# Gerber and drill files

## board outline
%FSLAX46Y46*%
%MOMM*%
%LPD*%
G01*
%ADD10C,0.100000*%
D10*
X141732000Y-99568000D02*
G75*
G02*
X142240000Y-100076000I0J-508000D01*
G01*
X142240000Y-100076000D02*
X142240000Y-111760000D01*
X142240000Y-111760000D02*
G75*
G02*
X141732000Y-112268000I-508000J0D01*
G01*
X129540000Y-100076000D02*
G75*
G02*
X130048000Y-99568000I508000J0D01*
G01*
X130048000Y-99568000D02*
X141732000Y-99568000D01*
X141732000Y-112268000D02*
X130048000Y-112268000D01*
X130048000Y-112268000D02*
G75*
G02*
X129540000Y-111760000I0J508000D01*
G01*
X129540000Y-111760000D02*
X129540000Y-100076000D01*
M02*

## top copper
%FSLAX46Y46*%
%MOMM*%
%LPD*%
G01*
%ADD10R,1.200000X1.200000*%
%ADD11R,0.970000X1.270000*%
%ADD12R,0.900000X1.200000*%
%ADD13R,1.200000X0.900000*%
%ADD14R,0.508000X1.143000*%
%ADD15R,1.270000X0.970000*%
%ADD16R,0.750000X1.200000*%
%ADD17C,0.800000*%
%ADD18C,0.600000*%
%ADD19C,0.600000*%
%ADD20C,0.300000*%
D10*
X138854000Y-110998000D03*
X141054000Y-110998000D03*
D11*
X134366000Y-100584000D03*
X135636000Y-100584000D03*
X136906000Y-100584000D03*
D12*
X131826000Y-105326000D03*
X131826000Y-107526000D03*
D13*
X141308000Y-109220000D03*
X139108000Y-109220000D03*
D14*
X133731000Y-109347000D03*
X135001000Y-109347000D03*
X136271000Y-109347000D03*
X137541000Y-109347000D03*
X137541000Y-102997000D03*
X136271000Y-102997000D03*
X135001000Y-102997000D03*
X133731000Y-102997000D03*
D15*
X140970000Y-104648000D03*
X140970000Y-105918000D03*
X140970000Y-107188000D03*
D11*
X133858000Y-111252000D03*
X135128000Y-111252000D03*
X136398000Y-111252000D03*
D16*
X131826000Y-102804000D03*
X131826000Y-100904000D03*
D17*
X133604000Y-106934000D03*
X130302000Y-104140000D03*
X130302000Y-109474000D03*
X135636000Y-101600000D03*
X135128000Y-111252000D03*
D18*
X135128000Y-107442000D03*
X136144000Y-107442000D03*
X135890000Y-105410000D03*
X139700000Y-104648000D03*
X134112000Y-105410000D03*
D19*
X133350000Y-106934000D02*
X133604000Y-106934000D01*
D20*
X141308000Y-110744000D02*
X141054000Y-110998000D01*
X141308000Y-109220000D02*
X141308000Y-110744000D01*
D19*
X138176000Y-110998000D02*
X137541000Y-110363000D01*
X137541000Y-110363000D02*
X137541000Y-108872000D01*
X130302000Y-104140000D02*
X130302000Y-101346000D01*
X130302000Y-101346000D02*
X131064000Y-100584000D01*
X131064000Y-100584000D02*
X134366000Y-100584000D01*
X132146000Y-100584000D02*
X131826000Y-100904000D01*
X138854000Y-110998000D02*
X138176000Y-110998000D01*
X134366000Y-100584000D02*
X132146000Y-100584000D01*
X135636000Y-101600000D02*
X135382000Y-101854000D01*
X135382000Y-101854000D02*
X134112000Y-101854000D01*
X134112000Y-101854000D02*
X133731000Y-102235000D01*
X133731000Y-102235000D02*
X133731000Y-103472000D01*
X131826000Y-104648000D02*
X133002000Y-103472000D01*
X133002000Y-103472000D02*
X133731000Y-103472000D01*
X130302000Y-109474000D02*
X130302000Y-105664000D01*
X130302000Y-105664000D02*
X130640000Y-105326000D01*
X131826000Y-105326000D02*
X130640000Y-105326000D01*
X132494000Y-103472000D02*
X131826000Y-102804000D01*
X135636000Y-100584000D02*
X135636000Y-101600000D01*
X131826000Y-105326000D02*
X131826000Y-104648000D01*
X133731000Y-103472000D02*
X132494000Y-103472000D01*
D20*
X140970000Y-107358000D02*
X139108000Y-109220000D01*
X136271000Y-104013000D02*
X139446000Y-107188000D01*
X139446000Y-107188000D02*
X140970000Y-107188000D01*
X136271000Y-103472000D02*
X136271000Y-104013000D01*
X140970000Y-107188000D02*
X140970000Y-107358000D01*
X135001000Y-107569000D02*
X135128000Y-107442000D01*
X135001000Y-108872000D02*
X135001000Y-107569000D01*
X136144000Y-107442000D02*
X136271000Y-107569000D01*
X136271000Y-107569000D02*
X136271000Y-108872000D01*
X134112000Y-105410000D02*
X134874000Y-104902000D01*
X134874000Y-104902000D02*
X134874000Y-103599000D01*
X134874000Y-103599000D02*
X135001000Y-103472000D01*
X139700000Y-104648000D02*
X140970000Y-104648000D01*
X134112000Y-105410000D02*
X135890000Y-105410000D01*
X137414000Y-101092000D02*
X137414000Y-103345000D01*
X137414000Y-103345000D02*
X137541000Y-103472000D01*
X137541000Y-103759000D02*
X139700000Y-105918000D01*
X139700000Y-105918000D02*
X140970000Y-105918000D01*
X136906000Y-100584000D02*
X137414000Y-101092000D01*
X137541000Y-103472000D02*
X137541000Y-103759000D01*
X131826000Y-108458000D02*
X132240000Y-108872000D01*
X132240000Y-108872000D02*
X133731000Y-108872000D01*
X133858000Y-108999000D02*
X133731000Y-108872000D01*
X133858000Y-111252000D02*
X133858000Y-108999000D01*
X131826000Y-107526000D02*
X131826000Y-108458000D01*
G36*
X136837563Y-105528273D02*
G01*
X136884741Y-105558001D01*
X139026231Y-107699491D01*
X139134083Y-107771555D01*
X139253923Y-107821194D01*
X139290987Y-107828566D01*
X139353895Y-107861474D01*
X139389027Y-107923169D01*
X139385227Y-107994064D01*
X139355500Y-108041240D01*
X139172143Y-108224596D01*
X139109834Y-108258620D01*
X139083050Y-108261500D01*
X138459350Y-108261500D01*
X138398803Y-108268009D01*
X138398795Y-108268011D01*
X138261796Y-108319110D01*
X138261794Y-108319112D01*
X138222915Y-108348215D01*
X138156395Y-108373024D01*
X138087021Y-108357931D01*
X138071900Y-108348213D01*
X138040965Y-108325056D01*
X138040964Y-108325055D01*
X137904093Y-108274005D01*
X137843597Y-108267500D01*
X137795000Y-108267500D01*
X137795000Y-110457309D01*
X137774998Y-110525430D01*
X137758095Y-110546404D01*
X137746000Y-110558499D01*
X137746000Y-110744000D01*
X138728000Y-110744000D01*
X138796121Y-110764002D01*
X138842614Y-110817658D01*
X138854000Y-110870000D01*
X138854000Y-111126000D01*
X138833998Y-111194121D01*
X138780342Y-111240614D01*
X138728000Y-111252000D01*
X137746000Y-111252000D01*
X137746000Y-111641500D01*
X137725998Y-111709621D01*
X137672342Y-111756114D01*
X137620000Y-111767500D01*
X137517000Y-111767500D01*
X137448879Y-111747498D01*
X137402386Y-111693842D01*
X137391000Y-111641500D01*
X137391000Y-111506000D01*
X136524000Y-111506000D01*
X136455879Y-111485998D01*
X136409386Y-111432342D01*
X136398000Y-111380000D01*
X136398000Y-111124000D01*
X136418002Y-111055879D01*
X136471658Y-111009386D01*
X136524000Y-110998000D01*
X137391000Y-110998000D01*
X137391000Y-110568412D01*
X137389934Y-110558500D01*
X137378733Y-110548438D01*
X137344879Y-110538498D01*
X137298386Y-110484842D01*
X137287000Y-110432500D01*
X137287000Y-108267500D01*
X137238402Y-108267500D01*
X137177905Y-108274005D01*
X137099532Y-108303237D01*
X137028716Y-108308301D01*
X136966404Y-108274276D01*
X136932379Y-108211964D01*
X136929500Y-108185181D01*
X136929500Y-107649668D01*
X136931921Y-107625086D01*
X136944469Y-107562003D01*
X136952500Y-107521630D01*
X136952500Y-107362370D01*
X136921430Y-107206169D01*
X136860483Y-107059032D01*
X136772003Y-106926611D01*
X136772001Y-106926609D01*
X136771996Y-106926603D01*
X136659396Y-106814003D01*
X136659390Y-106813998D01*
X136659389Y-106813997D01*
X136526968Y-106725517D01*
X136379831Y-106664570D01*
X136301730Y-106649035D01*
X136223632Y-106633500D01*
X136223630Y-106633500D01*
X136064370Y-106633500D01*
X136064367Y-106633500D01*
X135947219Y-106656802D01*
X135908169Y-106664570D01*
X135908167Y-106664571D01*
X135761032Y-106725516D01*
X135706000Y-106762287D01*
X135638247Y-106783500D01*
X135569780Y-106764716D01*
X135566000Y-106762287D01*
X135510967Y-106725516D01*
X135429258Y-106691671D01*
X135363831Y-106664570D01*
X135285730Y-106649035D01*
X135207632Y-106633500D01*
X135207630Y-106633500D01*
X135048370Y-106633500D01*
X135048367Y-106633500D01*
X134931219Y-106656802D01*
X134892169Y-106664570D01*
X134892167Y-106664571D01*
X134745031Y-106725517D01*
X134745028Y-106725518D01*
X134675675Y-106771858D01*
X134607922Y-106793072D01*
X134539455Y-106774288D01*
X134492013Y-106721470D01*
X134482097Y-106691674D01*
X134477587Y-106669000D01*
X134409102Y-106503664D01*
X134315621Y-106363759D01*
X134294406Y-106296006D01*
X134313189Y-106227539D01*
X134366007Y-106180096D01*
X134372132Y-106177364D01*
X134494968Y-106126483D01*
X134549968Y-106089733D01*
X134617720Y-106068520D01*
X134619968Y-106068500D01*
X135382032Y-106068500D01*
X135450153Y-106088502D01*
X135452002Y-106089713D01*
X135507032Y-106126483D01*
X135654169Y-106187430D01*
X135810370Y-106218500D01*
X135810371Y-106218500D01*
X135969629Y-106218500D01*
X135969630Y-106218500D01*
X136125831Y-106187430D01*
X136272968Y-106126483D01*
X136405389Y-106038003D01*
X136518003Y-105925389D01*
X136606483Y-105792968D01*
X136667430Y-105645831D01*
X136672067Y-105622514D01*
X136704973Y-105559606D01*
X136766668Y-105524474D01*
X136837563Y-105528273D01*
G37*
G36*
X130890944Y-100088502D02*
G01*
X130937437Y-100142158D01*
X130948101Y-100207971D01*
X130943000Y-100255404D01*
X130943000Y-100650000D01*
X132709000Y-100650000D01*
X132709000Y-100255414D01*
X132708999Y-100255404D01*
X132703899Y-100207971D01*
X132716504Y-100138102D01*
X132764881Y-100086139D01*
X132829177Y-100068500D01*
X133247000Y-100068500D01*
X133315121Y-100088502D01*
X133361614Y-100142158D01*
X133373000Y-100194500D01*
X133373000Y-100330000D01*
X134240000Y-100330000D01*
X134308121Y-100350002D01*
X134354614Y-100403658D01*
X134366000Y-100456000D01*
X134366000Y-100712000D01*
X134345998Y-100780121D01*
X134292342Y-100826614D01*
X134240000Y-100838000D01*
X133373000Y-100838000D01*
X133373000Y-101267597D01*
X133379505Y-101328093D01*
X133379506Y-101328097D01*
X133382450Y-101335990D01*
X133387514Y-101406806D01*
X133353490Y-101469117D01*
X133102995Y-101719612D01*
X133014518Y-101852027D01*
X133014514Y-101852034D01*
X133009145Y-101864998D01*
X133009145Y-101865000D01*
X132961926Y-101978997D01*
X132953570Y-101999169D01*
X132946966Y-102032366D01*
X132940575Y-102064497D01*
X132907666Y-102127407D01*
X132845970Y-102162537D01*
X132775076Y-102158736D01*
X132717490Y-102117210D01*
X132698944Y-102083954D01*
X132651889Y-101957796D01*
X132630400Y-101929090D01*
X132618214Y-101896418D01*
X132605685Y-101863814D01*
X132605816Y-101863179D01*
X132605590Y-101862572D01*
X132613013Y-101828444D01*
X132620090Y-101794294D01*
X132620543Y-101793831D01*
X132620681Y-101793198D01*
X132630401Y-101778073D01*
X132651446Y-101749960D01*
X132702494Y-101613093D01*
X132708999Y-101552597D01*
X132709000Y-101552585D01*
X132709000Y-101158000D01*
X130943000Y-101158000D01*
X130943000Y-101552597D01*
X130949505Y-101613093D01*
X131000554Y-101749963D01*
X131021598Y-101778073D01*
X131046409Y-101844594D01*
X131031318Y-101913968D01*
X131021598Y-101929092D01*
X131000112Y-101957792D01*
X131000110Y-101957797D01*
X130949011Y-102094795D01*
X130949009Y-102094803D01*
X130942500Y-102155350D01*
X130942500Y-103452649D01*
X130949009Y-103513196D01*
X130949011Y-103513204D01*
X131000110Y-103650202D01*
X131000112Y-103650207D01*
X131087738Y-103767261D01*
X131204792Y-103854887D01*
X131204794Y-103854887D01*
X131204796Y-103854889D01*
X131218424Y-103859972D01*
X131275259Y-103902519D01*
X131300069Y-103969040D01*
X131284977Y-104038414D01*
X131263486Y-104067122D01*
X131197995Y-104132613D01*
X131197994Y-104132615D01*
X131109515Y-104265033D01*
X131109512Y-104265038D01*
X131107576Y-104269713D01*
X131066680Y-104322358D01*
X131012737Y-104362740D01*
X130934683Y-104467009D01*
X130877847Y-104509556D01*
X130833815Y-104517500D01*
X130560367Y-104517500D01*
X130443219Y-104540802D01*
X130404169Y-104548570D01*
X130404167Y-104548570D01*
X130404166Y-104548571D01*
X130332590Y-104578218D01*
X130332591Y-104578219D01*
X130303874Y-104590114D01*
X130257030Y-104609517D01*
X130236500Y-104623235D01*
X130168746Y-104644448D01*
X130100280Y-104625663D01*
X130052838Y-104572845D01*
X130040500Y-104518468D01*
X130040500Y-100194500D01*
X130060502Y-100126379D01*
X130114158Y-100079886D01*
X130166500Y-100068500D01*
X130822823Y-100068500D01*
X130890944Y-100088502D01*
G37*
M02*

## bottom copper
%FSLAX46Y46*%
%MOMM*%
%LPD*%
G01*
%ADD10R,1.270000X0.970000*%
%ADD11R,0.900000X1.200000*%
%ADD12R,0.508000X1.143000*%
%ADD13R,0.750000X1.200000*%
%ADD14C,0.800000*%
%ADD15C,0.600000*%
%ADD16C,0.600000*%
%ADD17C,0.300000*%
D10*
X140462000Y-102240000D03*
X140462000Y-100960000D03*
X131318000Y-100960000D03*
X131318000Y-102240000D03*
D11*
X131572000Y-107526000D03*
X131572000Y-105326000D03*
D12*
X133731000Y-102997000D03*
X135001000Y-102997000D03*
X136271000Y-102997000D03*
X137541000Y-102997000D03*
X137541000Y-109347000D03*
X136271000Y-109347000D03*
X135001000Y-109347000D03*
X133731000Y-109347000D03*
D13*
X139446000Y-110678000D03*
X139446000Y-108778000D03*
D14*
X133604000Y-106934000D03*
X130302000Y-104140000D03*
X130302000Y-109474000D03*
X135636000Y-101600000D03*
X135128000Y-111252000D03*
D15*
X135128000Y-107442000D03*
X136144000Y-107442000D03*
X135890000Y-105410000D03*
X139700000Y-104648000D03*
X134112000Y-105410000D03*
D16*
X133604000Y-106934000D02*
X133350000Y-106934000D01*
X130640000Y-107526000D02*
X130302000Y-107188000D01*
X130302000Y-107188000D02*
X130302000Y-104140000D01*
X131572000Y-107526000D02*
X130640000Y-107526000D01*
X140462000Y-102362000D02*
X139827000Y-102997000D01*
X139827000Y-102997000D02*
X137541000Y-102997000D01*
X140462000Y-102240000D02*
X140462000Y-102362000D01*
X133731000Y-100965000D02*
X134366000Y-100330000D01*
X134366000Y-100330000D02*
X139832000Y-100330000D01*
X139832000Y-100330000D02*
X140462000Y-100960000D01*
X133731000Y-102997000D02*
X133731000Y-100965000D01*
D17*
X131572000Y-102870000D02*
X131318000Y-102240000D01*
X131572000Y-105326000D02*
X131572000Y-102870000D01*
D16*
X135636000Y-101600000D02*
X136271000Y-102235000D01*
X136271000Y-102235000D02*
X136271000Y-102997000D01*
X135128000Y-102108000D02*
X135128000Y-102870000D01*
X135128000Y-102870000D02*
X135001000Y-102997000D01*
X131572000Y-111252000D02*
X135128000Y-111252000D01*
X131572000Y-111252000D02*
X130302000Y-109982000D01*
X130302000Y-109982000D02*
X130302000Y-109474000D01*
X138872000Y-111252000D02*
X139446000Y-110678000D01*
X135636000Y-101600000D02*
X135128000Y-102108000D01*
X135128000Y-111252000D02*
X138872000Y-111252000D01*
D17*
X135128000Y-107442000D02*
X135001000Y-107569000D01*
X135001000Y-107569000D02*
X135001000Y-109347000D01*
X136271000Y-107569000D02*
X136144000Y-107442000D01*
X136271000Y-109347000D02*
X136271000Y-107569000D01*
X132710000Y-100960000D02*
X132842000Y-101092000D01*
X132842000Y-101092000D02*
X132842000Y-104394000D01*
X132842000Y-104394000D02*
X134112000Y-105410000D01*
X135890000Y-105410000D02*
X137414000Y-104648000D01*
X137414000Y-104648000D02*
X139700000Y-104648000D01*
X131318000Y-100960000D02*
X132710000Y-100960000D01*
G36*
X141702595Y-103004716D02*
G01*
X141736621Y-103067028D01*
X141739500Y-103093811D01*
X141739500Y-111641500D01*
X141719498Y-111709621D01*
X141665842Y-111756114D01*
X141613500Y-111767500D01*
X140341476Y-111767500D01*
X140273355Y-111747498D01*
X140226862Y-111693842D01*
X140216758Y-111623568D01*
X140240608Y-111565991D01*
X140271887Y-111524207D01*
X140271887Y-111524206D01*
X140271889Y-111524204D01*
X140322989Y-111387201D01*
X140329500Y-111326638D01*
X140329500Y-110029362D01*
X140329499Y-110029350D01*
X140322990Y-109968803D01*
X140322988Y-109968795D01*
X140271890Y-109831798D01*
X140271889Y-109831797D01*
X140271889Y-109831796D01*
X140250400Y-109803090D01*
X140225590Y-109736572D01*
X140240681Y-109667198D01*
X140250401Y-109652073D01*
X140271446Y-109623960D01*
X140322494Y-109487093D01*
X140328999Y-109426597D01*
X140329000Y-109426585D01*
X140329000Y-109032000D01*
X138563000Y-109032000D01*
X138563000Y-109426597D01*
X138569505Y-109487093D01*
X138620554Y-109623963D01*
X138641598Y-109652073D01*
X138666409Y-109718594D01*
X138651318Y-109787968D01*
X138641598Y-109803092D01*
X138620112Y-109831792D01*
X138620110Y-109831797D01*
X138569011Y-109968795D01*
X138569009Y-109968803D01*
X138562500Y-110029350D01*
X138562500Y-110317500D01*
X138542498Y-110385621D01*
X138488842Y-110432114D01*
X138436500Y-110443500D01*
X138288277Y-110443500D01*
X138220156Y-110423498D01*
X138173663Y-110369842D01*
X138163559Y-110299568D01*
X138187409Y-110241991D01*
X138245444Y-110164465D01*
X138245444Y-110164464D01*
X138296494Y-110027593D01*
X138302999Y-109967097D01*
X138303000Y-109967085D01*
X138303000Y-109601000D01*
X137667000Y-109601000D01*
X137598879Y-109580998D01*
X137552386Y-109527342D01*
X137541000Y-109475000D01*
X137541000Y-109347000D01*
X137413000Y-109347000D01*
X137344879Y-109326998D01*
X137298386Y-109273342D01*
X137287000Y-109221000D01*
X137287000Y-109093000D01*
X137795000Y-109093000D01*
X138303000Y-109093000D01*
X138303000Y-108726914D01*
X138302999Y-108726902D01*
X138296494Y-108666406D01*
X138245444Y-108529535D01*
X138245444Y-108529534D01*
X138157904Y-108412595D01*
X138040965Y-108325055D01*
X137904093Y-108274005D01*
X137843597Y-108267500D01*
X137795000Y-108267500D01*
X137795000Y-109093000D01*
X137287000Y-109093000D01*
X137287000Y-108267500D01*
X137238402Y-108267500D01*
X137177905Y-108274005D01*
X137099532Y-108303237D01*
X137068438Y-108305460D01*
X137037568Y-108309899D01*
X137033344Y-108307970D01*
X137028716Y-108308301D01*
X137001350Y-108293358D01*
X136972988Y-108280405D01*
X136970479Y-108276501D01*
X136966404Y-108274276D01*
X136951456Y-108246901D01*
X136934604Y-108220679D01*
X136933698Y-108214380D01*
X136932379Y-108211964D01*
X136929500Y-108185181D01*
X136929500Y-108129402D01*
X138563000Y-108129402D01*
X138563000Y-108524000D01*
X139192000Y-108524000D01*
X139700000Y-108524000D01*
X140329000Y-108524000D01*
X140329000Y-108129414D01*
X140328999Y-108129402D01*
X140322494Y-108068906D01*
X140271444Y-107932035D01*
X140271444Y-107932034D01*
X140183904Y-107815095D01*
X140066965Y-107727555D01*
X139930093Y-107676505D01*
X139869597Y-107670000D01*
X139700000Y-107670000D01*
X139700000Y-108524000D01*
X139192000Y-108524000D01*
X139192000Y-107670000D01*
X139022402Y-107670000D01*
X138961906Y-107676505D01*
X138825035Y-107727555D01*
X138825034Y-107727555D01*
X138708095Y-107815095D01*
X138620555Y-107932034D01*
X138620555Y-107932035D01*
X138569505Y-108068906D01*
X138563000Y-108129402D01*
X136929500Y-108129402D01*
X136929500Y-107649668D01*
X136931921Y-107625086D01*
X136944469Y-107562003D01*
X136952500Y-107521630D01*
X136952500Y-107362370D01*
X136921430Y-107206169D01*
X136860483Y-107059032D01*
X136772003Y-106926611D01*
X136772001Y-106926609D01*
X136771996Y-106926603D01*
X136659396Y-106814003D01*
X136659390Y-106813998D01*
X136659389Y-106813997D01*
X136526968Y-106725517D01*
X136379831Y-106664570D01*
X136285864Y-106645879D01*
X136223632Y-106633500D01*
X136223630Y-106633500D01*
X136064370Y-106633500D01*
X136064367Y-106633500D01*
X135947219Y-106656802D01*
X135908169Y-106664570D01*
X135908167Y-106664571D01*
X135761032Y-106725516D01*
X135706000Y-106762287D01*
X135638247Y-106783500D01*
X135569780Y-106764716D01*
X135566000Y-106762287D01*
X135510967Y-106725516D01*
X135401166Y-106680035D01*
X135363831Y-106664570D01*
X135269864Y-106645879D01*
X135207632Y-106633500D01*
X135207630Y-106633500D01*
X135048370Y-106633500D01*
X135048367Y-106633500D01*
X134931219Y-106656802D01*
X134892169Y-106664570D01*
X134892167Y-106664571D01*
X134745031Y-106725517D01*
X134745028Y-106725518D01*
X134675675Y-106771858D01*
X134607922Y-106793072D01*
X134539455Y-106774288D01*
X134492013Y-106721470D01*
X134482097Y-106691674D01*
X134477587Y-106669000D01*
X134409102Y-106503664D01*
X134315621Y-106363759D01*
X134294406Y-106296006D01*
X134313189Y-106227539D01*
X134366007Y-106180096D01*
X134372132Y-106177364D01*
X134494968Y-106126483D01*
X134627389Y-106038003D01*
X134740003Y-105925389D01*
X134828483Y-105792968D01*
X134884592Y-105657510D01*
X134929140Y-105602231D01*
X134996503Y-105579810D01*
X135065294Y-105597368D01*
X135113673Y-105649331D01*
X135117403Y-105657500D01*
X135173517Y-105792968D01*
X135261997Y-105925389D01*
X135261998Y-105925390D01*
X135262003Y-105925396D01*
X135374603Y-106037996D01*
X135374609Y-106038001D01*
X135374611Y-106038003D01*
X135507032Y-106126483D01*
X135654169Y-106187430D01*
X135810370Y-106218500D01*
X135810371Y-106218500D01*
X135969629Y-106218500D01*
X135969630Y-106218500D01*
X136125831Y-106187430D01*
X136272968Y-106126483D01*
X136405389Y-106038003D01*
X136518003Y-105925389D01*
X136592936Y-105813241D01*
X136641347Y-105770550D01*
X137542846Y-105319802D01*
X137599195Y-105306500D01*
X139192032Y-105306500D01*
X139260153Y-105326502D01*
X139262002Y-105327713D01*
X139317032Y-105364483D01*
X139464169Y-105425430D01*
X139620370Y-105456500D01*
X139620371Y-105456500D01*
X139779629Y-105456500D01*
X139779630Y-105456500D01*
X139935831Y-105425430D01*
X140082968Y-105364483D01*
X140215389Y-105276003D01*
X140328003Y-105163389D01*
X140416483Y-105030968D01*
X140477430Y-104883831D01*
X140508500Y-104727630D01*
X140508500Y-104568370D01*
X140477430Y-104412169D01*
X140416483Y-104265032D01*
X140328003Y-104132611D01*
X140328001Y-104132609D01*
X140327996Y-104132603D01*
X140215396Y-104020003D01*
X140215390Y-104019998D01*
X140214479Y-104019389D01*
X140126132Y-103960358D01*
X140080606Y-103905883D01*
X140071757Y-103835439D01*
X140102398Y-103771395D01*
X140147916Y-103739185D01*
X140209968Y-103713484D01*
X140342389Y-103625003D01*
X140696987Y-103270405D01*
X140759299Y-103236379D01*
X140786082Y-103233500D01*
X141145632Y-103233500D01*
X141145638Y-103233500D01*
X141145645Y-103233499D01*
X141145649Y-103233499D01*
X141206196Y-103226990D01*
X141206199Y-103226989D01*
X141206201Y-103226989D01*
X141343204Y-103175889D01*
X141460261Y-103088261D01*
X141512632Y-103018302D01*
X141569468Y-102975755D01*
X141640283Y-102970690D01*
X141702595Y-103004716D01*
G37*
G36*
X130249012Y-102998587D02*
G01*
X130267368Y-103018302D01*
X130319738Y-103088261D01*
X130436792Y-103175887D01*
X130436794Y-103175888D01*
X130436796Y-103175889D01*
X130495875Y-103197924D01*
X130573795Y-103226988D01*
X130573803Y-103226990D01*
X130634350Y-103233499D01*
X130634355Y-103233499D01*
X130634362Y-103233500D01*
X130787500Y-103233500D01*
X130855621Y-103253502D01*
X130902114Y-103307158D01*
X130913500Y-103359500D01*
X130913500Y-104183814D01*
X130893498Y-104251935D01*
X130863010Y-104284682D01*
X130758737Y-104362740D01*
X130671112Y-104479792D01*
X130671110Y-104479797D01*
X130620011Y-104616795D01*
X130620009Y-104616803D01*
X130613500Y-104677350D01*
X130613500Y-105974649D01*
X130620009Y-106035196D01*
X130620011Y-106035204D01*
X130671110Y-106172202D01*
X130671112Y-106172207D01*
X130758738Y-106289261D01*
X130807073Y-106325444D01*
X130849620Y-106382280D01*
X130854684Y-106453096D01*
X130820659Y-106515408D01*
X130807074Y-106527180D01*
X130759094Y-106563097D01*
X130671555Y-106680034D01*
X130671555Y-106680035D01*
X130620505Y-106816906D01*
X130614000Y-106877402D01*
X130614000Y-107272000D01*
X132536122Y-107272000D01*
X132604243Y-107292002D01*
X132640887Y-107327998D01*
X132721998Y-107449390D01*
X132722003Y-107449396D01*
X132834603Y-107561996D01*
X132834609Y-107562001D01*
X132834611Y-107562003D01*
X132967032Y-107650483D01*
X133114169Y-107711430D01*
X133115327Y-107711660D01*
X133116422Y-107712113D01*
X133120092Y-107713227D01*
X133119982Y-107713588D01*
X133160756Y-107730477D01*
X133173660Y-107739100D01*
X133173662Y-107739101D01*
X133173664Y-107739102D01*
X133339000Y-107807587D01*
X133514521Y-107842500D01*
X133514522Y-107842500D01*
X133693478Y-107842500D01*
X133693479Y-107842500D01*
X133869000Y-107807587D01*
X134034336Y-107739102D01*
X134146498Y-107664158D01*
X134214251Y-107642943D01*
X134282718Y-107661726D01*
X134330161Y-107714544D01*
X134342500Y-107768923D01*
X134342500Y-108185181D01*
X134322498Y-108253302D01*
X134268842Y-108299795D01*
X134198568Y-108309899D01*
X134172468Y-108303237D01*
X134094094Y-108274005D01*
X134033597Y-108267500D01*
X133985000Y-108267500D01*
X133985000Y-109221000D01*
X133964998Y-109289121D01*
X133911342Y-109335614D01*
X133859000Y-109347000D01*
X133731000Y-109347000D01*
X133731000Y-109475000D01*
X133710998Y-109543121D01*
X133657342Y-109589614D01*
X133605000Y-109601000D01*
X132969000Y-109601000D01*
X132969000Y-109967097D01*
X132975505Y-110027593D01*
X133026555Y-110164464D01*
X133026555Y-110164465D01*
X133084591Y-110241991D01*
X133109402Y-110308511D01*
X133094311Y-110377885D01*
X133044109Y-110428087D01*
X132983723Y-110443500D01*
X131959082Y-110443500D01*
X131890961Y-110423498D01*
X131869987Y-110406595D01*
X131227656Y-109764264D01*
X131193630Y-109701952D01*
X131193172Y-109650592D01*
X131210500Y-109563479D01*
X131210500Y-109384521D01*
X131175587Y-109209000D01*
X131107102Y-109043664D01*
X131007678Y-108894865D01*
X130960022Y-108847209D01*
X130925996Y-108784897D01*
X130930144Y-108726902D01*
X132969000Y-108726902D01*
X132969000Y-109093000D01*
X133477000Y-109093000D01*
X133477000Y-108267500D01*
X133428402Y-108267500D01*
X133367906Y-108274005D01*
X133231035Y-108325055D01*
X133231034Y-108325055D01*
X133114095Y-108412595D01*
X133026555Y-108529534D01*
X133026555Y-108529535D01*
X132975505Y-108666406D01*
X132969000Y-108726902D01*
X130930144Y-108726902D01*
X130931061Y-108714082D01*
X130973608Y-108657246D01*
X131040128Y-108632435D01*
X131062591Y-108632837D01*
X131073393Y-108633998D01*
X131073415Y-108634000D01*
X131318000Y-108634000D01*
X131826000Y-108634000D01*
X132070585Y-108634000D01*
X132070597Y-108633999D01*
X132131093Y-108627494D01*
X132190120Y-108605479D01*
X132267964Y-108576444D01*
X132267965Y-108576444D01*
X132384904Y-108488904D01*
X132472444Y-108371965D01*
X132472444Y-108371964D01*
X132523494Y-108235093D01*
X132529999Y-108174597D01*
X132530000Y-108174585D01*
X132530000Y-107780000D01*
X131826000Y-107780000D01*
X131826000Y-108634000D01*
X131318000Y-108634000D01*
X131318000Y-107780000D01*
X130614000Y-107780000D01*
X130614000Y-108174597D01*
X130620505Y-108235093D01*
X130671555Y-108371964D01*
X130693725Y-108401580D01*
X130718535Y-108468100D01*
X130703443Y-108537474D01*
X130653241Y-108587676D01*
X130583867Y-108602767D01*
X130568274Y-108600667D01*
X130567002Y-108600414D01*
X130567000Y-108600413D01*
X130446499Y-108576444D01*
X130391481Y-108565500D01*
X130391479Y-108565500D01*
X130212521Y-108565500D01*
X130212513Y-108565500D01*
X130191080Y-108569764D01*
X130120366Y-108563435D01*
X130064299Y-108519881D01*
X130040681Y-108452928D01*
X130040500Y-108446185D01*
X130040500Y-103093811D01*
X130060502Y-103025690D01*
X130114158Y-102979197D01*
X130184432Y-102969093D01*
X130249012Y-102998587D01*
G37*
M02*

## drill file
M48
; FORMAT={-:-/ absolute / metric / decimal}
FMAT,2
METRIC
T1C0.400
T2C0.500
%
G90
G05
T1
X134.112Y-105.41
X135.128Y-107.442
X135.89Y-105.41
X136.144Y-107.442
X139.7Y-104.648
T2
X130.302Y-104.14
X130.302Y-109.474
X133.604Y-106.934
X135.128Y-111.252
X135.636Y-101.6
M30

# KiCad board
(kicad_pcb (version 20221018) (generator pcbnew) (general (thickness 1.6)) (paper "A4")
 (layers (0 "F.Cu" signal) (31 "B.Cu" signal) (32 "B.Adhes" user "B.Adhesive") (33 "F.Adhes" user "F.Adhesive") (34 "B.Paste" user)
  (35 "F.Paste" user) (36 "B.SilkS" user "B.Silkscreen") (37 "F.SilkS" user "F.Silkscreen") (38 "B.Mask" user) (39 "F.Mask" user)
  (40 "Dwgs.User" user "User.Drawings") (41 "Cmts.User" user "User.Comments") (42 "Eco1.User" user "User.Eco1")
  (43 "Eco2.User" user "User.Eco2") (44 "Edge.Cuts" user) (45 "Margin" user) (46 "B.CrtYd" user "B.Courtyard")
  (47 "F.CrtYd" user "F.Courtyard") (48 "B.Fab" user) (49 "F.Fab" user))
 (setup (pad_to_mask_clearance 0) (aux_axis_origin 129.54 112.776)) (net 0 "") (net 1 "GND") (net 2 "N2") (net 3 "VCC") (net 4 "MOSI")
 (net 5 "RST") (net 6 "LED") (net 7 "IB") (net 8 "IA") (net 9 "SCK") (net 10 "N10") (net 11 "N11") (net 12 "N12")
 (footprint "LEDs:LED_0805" (layer "F.Cu") (at 139.954 110.998)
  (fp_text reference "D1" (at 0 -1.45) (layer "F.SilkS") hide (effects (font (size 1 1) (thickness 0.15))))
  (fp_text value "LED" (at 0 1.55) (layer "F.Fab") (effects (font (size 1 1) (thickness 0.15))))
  (pad "1" smd rect (at -1.1 0 180) (size 1.2 1.2) (layers "F.Cu" "F.Paste" "F.Mask") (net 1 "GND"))
  (pad "2" smd rect (at 1.1 0 180) (size 1.2 1.2) (layers "F.Cu" "F.Paste" "F.Mask") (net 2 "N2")))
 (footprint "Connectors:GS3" (layer "F.Cu") (at 135.636 100.584 90)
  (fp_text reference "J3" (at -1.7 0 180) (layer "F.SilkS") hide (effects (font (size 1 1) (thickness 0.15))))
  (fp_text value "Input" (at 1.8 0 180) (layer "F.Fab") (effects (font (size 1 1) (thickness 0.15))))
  (pad "1" smd rect (at 0 -1.27 90) (size 1.27 0.97) (layers "F.Cu" "F.Paste" "F.Mask") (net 1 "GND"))
  (pad "2" smd rect (at 0 0 90) (size 1.27 0.97) (layers "F.Cu" "F.Paste" "F.Mask") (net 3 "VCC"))
  (pad "3" smd rect (at 0 1.27 90) (size 1.27 0.97) (layers "F.Cu" "F.Paste" "F.Mask") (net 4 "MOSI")))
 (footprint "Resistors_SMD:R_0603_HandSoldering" (layer "F.Cu") (at 131.826 106.426 -90)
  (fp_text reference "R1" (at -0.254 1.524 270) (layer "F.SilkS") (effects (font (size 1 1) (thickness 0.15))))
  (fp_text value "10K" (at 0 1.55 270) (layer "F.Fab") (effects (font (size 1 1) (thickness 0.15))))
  (pad "1" smd rect (at -1.1 0 270) (size 1.2 0.9) (layers "F.Cu" "F.Paste" "F.Mask") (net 3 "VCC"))
  (pad "2" smd rect (at 1.1 0 270) (size 1.2 0.9) (layers "F.Cu" "F.Paste" "F.Mask") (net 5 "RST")))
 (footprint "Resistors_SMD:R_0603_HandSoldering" (layer "F.Cu") (at 140.208 109.22 180)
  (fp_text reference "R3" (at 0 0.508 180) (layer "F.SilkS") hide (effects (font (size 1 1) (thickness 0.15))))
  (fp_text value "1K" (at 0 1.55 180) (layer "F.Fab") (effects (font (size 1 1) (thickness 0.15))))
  (pad "1" smd rect (at -1.1 0 180) (size 1.2 0.9) (layers "F.Cu" "F.Paste" "F.Mask") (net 2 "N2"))
  (pad "2" smd rect (at 1.1 0 180) (size 1.2 0.9) (layers "F.Cu" "F.Paste" "F.Mask") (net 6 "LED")))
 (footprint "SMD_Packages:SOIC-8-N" (layer "F.Cu") (at 135.636 106.172)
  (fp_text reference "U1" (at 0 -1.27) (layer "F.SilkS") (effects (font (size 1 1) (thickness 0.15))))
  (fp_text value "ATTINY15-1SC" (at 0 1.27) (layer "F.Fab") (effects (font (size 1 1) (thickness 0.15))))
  (pad "1" smd rect (at -1.905 3.175) (size 0.508 1.143) (layers "F.Cu" "F.Paste" "F.Mask") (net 5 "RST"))
  (pad "2" smd rect (at -0.635 3.175) (size 0.508 1.143) (layers "F.Cu" "F.Paste" "F.Mask") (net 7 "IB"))
  (pad "3" smd rect (at 0.635 3.175) (size 0.508 1.143) (layers "F.Cu" "F.Paste" "F.Mask") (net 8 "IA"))
  (pad "4" smd rect (at 1.905 3.175) (size 0.508 1.143) (layers "F.Cu" "F.Paste" "F.Mask") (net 1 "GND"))
  (pad "5" smd rect (at 1.905 -3.175) (size 0.508 1.143) (layers "F.Cu" "F.Paste" "F.Mask") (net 4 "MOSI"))
  (pad "6" smd rect (at 0.635 -3.175) (size 0.508 1.143) (layers "F.Cu" "F.Paste" "F.Mask") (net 6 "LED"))
  (pad "7" smd rect (at -0.635 -3.175) (size 0.508 1.143) (layers "F.Cu" "F.Paste" "F.Mask") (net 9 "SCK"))
  (pad "8" smd rect (at -1.905 -3.175) (size 0.508 1.143) (layers "F.Cu" "F.Paste" "F.Mask") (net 3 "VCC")))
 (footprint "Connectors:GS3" (layer "F.Cu") (at 140.97 105.918)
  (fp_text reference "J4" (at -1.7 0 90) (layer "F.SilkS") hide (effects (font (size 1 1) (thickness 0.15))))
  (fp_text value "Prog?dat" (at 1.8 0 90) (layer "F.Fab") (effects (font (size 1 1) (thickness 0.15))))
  (pad "1" smd rect (at 0 -1.27) (size 1.27 0.97) (layers "F.Cu" "F.Paste" "F.Mask") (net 9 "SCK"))
  (pad "2" smd rect (at 0 0) (size 1.27 0.97) (layers "F.Cu" "F.Paste" "F.Mask") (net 4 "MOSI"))
  (pad "3" smd rect (at 0 1.27) (size 1.27 0.97) (layers "F.Cu" "F.Paste" "F.Mask") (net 6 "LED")))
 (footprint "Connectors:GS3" (layer "F.Cu") (at 135.128 111.252 90)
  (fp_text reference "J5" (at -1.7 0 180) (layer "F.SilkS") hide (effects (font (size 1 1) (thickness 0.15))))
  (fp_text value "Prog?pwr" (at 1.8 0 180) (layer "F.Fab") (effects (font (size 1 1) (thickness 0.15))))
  (pad "1" smd rect (at 0 -1.27 90) (size 1.27 0.97) (layers "F.Cu" "F.Paste" "F.Mask") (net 5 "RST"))
  (pad "2" smd rect (at 0 0 90) (size 1.27 0.97) (layers "F.Cu" "F.Paste" "F.Mask") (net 3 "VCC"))
  (pad "3" smd rect (at 0 1.27 90) (size 1.27 0.97) (layers "F.Cu" "F.Paste" "F.Mask") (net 1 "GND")))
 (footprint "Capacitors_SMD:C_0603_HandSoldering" (layer "F.Cu") (at 131.826 101.854 90)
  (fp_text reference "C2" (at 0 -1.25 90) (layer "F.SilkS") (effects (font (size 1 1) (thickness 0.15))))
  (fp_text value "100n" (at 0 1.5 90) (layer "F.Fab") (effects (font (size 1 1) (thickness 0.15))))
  (pad "1" smd rect (at -0.95 0 90) (size 1.2 0.75) (layers "F.Cu" "F.Paste" "F.Mask") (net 3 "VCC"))
  (pad "2" smd rect (at 0.95 0 90) (size 1.2 0.75) (layers "F.Cu" "F.Paste" "F.Mask") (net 1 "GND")))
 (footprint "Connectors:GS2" (layer "B.Cu") (at 140.462 101.6)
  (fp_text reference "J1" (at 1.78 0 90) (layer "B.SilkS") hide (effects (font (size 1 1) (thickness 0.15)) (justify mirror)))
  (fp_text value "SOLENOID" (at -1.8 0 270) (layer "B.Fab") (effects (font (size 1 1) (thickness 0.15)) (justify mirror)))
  (pad "1" smd rect (at 0 0.64) (size 1.27 0.97) (layers "B.Cu" "B.Paste" "B.Mask") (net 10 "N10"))
  (pad "2" smd rect (at 0 -0.64) (size 1.27 0.97) (layers "B.Cu" "B.Paste" "B.Mask") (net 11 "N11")))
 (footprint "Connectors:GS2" (layer "B.Cu") (at 131.318 101.6 180)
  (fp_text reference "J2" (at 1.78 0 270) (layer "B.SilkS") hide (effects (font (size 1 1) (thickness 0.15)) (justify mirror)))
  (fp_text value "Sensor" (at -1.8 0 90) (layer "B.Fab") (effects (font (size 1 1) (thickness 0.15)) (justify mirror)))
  (pad "1" smd rect (at 0 0.64 180) (size 1.27 0.97) (layers "B.Cu" "B.Paste" "B.Mask") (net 9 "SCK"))
  (pad "2" smd rect (at 0 -0.64 180) (size 1.27 0.97) (layers "B.Cu" "B.Paste" "B.Mask") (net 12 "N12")))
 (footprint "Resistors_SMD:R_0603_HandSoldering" (layer "B.Cu") (at 131.572 106.426 90)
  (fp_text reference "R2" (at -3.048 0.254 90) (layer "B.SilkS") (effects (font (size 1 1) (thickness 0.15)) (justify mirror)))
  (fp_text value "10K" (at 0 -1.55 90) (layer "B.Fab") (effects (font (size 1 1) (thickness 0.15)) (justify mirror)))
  (pad "1" smd rect (at -1.1 0 90) (size 1.2 0.9) (layers "B.Cu" "B.Paste" "B.Mask") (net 1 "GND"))
  (pad "2" smd rect (at 1.1 0 90) (size 1.2 0.9) (layers "B.Cu" "B.Paste" "B.Mask") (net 12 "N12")))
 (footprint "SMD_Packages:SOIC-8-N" (layer "B.Cu") (at 135.636 106.172)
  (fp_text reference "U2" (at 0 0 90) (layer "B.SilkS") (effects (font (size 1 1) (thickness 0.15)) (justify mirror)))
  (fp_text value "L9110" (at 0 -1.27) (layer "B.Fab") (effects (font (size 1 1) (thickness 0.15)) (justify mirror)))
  (pad "1" smd rect (at -1.905 -3.175) (size 0.508 1.143) (layers "B.Cu" "B.Paste" "B.Mask") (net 11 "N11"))
  (pad "2" smd rect (at -0.635 -3.175) (size 0.508 1.143) (layers "B.Cu" "B.Paste" "B.Mask") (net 3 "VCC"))
  (pad "3" smd rect (at 0.635 -3.175) (size 0.508 1.143) (layers "B.Cu" "B.Paste" "B.Mask") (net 3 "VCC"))
  (pad "4" smd rect (at 1.905 -3.175) (size 0.508 1.143) (layers "B.Cu" "B.Paste" "B.Mask") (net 10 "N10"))
  (pad "5" smd rect (at 1.905 3.175) (size 0.508 1.143) (layers "B.Cu" "B.Paste" "B.Mask") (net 1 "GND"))
  (pad "6" smd rect (at 0.635 3.175) (size 0.508 1.143) (layers "B.Cu" "B.Paste" "B.Mask") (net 8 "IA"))
  (pad "7" smd rect (at -0.635 3.175) (size 0.508 1.143) (layers "B.Cu" "B.Paste" "B.Mask") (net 7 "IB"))
  (pad "8" smd rect (at -1.905 3.175) (size 0.508 1.143) (layers "B.Cu" "B.Paste" "B.Mask") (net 1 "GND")))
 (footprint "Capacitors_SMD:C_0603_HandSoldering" (layer "B.Cu") (at 139.446 109.728 90)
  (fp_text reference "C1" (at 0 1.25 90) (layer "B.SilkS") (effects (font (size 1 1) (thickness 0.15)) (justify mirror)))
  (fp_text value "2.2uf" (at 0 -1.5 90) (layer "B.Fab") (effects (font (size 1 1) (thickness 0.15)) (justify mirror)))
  (pad "1" smd rect (at -0.95 0 90) (size 1.2 0.75) (layers "B.Cu" "B.Paste" "B.Mask") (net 3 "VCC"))
  (pad "2" smd rect (at 0.95 0 90) (size 1.2 0.75) (layers "B.Cu" "B.Paste" "B.Mask") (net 1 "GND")))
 (gr_arc (start 141.732 99.568) (mid 142.09121 99.71679) (end 142.24 100.076) (stroke (width 0.1) (type solid)) (layer "Edge.Cuts"))
 (gr_line (start 142.24 100.076) (end 142.24 111.76) (stroke (width 0.1) (type solid)) (layer "Edge.Cuts"))
 (gr_arc (start 142.24 111.76) (mid 142.09121 112.11921) (end 141.732 112.268) (stroke (width 0.1) (type solid)) (layer "Edge.Cuts"))
 (gr_arc (start 129.54 100.076) (mid 129.68879 99.71679) (end 130.048 99.568) (stroke (width 0.1) (type solid)) (layer "Edge.Cuts"))
 (gr_line (start 130.048 99.568) (end 141.732 99.568) (stroke (width 0.1) (type solid)) (layer "Edge.Cuts"))
 (gr_line (start 141.732 112.268) (end 130.048 112.268) (stroke (width 0.1) (type solid)) (layer "Edge.Cuts"))
 (gr_arc (start 130.048 112.268) (mid 129.68879 112.11921) (end 129.54 111.76) (stroke (width 0.1) (type solid)) (layer "Edge.Cuts"))
 (gr_line (start 129.54 111.76) (end 129.54 100.076) (stroke (width 0.1) (type solid)) (layer "Edge.Cuts"))
 (segment (start 133.35 106.934) (end 133.604 106.934) (width 0.6) (layer "F.Cu") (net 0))
 (via (at 133.604 106.934) (size 0.8) (drill 0.5) (layers "F.Cu" "B.Cu") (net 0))
 (segment (start 133.604 106.934) (end 133.35 106.934) (width 0.6) (layer "B.Cu") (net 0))
 (segment (start 141.308 110.744) (end 141.054 110.998) (width 0.3) (layer "F.Cu") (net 2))
 (segment (start 141.308 109.22) (end 141.308 110.744) (width 0.3) (layer "F.Cu") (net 2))
 (segment (start 138.176 110.998) (end 137.541 110.363) (width 0.6) (layer "F.Cu") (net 1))
 (segment (start 137.541 110.363) (end 137.541 108.872) (width 0.6) (layer "F.Cu") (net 1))
 (segment (start 130.302 104.14) (end 130.302 101.346) (width 0.6) (layer "F.Cu") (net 1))
 (segment (start 130.302 101.346) (end 131.064 100.584) (width 0.6) (layer "F.Cu") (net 1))
 (segment (start 131.064 100.584) (end 134.366 100.584) (width 0.6) (layer "F.Cu") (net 1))
 (segment (start 132.146 100.584) (end 131.826 100.904) (width 0.6) (layer "F.Cu") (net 1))
 (segment (start 138.854 110.998) (end 138.176 110.998) (width 0.6) (layer "F.Cu") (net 1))
 (segment (start 134.366 100.584) (end 132.146 100.584) (width 0.6) (layer "F.Cu") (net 1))
 (via (at 130.302 104.14) (size 0.8) (drill 0.5) (layers "F.Cu" "B.Cu") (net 1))
 (segment (start 130.64 107.526) (end 130.302 107.188) (width 0.6) (layer "B.Cu") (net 1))
 (segment (start 130.302 107.188) (end 130.302 104.14) (width 0.6) (layer "B.Cu") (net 1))
 (segment (start 131.572 107.526) (end 130.64 107.526) (width 0.6) (layer "B.Cu") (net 1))
 (segment (start 140.462 102.362) (end 139.827 102.997) (width 0.6) (layer "B.Cu") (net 10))
 (segment (start 139.827 102.997) (end 137.541 102.997) (width 0.6) (layer "B.Cu") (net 10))
 (segment (start 140.462 102.24) (end 140.462 102.362) (width 0.6) (layer "B.Cu") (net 10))
 (segment (start 133.731 100.965) (end 134.366 100.33) (width 0.6) (layer "B.Cu") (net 11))
 (segment (start 134.366 100.33) (end 139.832 100.33) (width 0.6) (layer "B.Cu") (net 11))
 (segment (start 139.832 100.33) (end 140.462 100.96) (width 0.6) (layer "B.Cu") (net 11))
 (segment (start 133.731 102.997) (end 133.731 100.965) (width 0.6) (layer "B.Cu") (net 11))
 (segment (start 131.572 102.87) (end 131.318 102.24) (width 0.3) (layer "B.Cu") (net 12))
 (segment (start 131.572 105.326) (end 131.572 102.87) (width 0.3) (layer "B.Cu") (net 12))
 (segment (start 135.636 101.6) (end 135.382 101.854) (width 0.6) (layer "F.Cu") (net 3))
 (segment (start 135.382 101.854) (end 134.112 101.854) (width 0.6) (layer "F.Cu") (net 3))
 (segment (start 134.112 101.854) (end 133.731 102.235) (width 0.6) (layer "F.Cu") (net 3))
 (segment (start 133.731 102.235) (end 133.731 103.472) (width 0.6) (layer "F.Cu") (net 3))
 (segment (start 131.826 104.648) (end 133.002 103.472) (width 0.6) (layer "F.Cu") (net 3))
 (segment (start 133.002 103.472) (end 133.731 103.472) (width 0.6) (layer "F.Cu") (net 3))
 (segment (start 130.302 109.474) (end 130.302 105.664) (width 0.6) (layer "F.Cu") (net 3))
 (segment (start 130.302 105.664) (end 130.64 105.326) (width 0.6) (layer "F.Cu") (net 3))
 (segment (start 131.826 105.326) (end 130.64 105.326) (width 0.6) (layer "F.Cu") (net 3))
 (segment (start 132.494 103.472) (end 131.826 102.804) (width 0.6) (layer "F.Cu") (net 3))
 (segment (start 135.636 100.584) (end 135.636 101.6) (width 0.6) (layer "F.Cu") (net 3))
 (segment (start 131.826 105.326) (end 131.826 104.648) (width 0.6) (layer "F.Cu") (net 3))
 (segment (start 133.731 103.472) (end 132.494 103.472) (width 0.6) (layer "F.Cu") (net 3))
 (via (at 130.302 109.474) (size 0.8) (drill 0.5) (layers "F.Cu" "B.Cu") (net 3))
 (via (at 135.636 101.6) (size 0.8) (drill 0.5) (layers "F.Cu" "B.Cu") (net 3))
 (via (at 135.128 111.252) (size 0.8) (drill 0.5) (layers "F.Cu" "B.Cu") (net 3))
 (segment (start 135.636 101.6) (end 136.271 102.235) (width 0.6) (layer "B.Cu") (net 3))
 (segment (start 136.271 102.235) (end 136.271 102.997) (width 0.6) (layer "B.Cu") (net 3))
 (segment (start 135.128 102.108) (end 135.128 102.87) (width 0.6) (layer "B.Cu") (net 3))
 (segment (start 135.128 102.87) (end 135.001 102.997) (width 0.6) (layer "B.Cu") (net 3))
 (segment (start 131.572 111.252) (end 135.128 111.252) (width 0.6) (layer "B.Cu") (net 3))
 (segment (start 131.572 111.252) (end 130.302 109.982) (width 0.6) (layer "B.Cu") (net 3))
 (segment (start 130.302 109.982) (end 130.302 109.474) (width 0.6) (layer "B.Cu") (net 3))
 (segment (start 138.872 111.252) (end 139.446 110.678) (width 0.6) (layer "B.Cu") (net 3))
 (segment (start 135.636 101.6) (end 135.128 102.108) (width 0.6) (layer "B.Cu") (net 3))
 (segment (start 135.128 111.252) (end 138.872 111.252) (width 0.6) (layer "B.Cu") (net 3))
 (segment (start 140.97 107.358) (end 139.108 109.22) (width 0.3) (layer "F.Cu") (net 6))
 (segment (start 136.271 104.013) (end 139.446 107.188) (width 0.3) (layer "F.Cu") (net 6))
 (segment (start 139.446 107.188) (end 140.97 107.188) (width 0.3) (layer "F.Cu") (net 6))
 (segment (start 136.271 103.472) (end 136.271 104.013) (width 0.3) (layer "F.Cu") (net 6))
 (segment (start 140.97 107.188) (end 140.97 107.358) (width 0.3) (layer "F.Cu") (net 6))
 (segment (start 135.001 107.569) (end 135.128 107.442) (width 0.3) (layer "F.Cu") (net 7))
 (segment (start 135.001 108.872) (end 135.001 107.569) (width 0.3) (layer "F.Cu") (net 7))
 (via (at 135.128 107.442) (size 0.6) (drill 0.4) (layers "F.Cu" "B.Cu") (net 7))
 (segment (start 135.128 107.442) (end 135.001 107.569) (width 0.3) (layer "B.Cu") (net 7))
 (segment (start 135.001 107.569) (end 135.001 109.347) (width 0.3) (layer "B.Cu") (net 7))
 (segment (start 136.144 107.442) (end 136.271 107.569) (width 0.3) (layer "F.Cu") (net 8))
 (segment (start 136.271 107.569) (end 136.271 108.872) (width 0.3) (layer "F.Cu") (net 8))
 (via (at 136.144 107.442) (size 0.6) (drill 0.4) (layers "F.Cu" "B.Cu") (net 8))
 (segment (start 136.271 107.569) (end 136.144 107.442) (width 0.3) (layer "B.Cu") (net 8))
 (segment (start 136.271 109.347) (end 136.271 107.569) (width 0.3) (layer "B.Cu") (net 8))
 (segment (start 134.112 105.41) (end 134.874 104.902) (width 0.3) (layer "F.Cu") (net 9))
 (segment (start 134.874 104.902) (end 134.874 103.599) (width 0.3) (layer "F.Cu") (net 9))
 (segment (start 134.874 103.599) (end 135.001 103.472) (width 0.3) (layer "F.Cu") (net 9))
 (segment (start 139.7 104.648) (end 140.97 104.648) (width 0.3) (layer "F.Cu") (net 9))
 (segment (start 134.112 105.41) (end 135.89 105.41) (width 0.3) (layer "F.Cu") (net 9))
 (via (at 135.89 105.41) (size 0.6) (drill 0.4) (layers "F.Cu" "B.Cu") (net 9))
 (via (at 139.7 104.648) (size 0.6) (drill 0.4) (layers "F.Cu" "B.Cu") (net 9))
 (via (at 134.112 105.41) (size 0.6) (drill 0.4) (layers "F.Cu" "B.Cu") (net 9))
 (segment (start 132.71 100.96) (end 132.842 101.092) (width 0.3) (layer "B.Cu") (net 9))
 (segment (start 132.842 101.092) (end 132.842 104.394) (width 0.3) (layer "B.Cu") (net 9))
 (segment (start 132.842 104.394) (end 134.112 105.41) (width 0.3) (layer "B.Cu") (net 9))
 (segment (start 135.89 105.41) (end 137.414 104.648) (width 0.3) (layer "B.Cu") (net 9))
 (segment (start 137.414 104.648) (end 139.7 104.648) (width 0.3) (layer "B.Cu") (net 9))
 (segment (start 131.318 100.96) (end 132.71 100.96) (width 0.3) (layer "B.Cu") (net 9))
 (segment (start 137.414 101.092) (end 137.414 103.345) (width 0.3) (layer "F.Cu") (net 4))
 (segment (start 137.414 103.345) (end 137.541 103.472) (width 0.3) (layer "F.Cu") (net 4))
 (segment (start 137.541 103.759) (end 139.7 105.918) (width 0.3) (layer "F.Cu") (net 4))
 (segment (start 139.7 105.918) (end 140.97 105.918) (width 0.3) (layer "F.Cu") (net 4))
 (segment (start 136.906 100.584) (end 137.414 101.092) (width 0.3) (layer "F.Cu") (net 4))
 (segment (start 137.541 103.472) (end 137.541 103.759) (width 0.3) (layer "F.Cu") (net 4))
 (segment (start 131.826 108.458) (end 132.24 108.872) (width 0.3) (layer "F.Cu") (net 5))
 (segment (start 132.24 108.872) (end 133.731 108.872) (width 0.3) (layer "F.Cu") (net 5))
 (segment (start 133.858 108.999) (end 133.731 108.872) (width 0.3) (layer "F.Cu") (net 5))
 (segment (start 133.858 111.252) (end 133.858 108.999) (width 0.3) (layer "F.Cu") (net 5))
 (segment (start 131.826 107.526) (end 131.826 108.458) (width 0.3) (layer "F.Cu") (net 5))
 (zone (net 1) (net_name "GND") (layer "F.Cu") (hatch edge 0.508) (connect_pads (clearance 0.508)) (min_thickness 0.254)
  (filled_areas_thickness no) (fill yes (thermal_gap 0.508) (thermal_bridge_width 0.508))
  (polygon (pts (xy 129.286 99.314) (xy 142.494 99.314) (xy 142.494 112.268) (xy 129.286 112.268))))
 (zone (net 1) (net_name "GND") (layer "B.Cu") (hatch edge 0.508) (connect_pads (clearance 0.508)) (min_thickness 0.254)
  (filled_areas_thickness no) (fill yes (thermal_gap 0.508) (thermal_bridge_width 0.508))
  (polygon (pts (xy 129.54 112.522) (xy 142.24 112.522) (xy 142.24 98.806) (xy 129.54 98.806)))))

